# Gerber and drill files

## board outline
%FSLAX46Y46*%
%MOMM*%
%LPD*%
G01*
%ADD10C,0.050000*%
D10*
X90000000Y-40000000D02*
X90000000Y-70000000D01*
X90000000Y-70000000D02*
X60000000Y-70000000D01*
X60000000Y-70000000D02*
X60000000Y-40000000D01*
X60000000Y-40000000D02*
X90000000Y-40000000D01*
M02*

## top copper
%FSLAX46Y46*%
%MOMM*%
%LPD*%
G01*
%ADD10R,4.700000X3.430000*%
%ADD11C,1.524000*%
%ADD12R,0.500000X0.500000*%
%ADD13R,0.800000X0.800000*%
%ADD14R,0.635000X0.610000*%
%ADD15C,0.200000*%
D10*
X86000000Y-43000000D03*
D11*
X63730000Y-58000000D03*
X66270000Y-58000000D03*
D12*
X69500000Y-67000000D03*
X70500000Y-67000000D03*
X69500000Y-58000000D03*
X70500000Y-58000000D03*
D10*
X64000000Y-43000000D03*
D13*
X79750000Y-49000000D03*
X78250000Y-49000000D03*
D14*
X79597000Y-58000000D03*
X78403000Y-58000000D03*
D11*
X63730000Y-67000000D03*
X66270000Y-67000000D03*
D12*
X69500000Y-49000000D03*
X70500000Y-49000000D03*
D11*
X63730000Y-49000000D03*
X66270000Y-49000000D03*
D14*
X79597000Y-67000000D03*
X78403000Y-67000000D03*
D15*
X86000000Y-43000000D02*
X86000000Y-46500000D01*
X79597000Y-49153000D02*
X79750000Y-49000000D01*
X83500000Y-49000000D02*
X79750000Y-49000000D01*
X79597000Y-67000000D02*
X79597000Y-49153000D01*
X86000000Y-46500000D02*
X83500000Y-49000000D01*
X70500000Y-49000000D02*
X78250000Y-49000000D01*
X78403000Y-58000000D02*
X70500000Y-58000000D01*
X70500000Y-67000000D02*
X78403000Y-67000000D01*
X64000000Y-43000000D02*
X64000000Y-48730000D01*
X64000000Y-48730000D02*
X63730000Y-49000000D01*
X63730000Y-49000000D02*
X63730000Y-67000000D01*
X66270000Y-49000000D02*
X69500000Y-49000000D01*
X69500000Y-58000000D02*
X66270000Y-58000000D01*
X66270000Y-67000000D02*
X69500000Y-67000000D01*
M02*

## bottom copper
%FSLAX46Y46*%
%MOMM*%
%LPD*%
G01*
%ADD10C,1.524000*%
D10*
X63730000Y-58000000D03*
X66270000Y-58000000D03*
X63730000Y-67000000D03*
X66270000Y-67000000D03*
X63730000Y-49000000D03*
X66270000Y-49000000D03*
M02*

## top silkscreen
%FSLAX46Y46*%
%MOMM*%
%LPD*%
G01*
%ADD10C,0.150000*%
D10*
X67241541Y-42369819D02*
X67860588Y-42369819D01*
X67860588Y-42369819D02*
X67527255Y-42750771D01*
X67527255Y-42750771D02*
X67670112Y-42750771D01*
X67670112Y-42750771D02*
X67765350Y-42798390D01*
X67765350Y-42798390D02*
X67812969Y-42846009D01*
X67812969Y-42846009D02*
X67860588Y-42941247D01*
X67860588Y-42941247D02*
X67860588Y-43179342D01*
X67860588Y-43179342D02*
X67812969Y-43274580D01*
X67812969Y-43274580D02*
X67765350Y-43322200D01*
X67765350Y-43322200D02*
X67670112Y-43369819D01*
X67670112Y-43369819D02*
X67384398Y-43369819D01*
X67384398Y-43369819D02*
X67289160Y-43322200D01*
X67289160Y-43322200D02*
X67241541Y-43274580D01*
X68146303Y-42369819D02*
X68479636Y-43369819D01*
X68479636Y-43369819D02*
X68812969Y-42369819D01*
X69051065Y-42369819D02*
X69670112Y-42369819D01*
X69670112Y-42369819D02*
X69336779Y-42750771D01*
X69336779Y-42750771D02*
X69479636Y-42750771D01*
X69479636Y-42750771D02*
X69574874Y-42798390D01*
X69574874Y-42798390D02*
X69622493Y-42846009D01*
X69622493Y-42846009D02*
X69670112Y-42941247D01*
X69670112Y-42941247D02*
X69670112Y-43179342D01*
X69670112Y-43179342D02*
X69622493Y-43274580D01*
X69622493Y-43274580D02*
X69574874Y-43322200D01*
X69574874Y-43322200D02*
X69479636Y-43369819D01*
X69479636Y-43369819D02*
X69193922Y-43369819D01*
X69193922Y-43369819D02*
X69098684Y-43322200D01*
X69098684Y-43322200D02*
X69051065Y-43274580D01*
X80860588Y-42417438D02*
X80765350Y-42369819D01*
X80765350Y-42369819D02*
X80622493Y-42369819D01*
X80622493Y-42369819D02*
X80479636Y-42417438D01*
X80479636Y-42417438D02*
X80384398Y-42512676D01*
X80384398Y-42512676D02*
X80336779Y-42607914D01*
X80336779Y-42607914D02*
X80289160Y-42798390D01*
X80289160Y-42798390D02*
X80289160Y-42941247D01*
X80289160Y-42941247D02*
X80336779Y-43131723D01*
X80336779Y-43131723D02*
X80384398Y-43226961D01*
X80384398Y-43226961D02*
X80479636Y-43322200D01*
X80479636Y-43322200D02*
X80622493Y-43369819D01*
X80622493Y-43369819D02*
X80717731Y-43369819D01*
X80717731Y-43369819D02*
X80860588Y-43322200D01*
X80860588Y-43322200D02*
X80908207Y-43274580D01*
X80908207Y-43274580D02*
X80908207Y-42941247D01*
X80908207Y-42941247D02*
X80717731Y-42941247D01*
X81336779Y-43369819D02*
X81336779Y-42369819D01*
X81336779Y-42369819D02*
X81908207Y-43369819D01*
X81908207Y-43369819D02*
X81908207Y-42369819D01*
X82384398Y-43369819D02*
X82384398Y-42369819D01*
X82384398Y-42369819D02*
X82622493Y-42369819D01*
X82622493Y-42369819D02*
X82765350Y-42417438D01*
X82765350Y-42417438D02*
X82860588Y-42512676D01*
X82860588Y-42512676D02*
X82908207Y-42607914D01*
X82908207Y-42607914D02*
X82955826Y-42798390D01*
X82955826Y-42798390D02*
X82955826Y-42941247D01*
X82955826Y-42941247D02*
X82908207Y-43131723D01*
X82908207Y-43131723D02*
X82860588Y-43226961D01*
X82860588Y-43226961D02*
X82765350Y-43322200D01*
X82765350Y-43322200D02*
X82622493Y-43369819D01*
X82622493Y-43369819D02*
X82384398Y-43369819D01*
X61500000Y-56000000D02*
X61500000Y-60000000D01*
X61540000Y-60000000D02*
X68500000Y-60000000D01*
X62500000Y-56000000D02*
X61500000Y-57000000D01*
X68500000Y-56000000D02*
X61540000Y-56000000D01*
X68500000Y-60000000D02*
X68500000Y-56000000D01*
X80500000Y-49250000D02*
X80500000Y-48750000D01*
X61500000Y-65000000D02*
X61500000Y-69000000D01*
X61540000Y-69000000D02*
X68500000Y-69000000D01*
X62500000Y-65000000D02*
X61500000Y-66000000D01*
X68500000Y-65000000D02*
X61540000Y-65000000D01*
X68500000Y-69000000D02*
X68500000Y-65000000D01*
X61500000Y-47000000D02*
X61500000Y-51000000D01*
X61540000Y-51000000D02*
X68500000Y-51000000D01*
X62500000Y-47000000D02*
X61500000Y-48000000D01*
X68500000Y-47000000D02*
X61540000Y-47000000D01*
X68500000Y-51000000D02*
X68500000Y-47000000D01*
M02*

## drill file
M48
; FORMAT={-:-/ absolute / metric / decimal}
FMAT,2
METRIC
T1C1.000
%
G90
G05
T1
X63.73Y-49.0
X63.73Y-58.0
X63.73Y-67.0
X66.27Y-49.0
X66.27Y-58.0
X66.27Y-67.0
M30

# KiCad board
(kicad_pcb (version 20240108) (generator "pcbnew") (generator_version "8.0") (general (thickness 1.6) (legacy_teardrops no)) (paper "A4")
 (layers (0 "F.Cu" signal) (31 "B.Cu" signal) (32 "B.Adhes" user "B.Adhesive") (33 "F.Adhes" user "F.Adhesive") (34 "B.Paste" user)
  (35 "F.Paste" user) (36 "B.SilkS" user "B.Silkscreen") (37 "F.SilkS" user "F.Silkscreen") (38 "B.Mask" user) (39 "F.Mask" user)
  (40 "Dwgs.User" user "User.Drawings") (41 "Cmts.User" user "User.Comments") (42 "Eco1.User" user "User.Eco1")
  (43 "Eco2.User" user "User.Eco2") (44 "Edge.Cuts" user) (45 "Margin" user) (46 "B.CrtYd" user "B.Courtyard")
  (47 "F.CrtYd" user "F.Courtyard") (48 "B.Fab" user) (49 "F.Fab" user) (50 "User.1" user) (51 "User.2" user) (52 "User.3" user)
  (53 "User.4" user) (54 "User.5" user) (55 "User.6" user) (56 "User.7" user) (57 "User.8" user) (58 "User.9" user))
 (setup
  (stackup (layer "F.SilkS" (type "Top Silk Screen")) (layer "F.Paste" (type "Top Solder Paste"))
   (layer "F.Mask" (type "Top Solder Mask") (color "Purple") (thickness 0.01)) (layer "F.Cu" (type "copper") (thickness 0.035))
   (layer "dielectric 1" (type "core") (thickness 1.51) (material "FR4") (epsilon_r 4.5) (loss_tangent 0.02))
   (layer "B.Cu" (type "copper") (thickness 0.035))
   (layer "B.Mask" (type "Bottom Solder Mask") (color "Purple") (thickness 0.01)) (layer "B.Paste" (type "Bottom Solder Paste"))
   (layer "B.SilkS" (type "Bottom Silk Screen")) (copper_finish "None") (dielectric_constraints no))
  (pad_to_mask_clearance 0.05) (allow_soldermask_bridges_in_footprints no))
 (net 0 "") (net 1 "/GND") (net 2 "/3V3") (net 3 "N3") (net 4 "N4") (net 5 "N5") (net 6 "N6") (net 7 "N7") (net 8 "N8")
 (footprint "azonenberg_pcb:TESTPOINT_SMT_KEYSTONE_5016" (layer "F.Cu") (at 86 43)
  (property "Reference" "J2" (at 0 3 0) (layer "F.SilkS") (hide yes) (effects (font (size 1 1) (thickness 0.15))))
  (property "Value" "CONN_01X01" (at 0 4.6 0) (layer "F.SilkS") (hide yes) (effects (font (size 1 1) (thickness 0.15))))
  (pad "1" smd rect (at 0 0) (size 4.7 3.43) (layers "F.Cu" "F.Paste" "F.Mask") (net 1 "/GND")))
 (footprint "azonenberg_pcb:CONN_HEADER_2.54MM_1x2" (layer "F.Cu") (at 65 58)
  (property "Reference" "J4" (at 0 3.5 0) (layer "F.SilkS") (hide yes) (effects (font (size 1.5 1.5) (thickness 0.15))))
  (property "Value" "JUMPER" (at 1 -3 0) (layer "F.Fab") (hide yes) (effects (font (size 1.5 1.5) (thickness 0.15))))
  (fp_line (start -3.5 -2) (end -3.5 2) (stroke (width 0.15) (type solid)) (layer "F.SilkS"))
  (fp_line (start -3.46 2) (end 3.5 2) (stroke (width 0.15) (type solid)) (layer "F.SilkS"))
  (fp_line (start -2.5 -2) (end -3.5 -1) (stroke (width 0.15) (type solid)) (layer "F.SilkS"))
  (fp_line (start 3.5 -2) (end -3.46 -2) (stroke (width 0.15) (type solid)) (layer "F.SilkS"))
  (fp_line (start 3.5 2) (end 3.5 -2) (stroke (width 0.15) (type solid)) (layer "F.SilkS"))
  (pad "1" thru_hole circle (at -1.27 0) (size 1.524 1.524) (drill 1) (layers "*.Cu" "*.Mask") (remove_unused_layers no) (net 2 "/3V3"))
  (pad "2" thru_hole circle (at 1.27 0) (size 1.524 1.524) (drill 1) (layers "*.Cu" "*.Mask") (remove_unused_layers no) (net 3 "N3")))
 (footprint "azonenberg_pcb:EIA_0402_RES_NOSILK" (layer "F.Cu") (at 70 67)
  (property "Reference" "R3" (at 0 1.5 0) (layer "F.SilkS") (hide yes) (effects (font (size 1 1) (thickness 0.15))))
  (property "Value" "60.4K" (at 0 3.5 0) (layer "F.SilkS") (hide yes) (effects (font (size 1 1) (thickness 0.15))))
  (pad "1" smd rect (at -0.5 0) (size 0.5 0.5) (layers "F.Cu" "F.Paste" "F.Mask") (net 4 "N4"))
  (pad "2" smd rect (at 0.5 0) (size 0.5 0.5) (layers "F.Cu" "F.Paste" "F.Mask") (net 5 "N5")))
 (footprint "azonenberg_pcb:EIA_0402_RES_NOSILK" (layer "F.Cu") (at 70 58)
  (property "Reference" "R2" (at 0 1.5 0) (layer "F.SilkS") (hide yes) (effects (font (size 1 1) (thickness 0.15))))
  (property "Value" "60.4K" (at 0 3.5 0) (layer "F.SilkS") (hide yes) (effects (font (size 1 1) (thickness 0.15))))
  (pad "1" smd rect (at -0.5 0) (size 0.5 0.5) (layers "F.Cu" "F.Paste" "F.Mask") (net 3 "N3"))
  (pad "2" smd rect (at 0.5 0) (size 0.5 0.5) (layers "F.Cu" "F.Paste" "F.Mask") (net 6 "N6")))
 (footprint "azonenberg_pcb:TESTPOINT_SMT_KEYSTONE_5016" (layer "F.Cu") (at 64 43)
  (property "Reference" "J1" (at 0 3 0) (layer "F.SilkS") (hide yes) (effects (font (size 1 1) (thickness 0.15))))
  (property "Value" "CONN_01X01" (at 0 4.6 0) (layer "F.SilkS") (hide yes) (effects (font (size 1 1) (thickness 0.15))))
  (pad "1" smd rect (at 0 0) (size 4.7 3.43) (layers "F.Cu" "F.Paste" "F.Mask") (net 2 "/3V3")))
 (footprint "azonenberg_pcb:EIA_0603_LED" (layer "F.Cu") (at 79 49 180)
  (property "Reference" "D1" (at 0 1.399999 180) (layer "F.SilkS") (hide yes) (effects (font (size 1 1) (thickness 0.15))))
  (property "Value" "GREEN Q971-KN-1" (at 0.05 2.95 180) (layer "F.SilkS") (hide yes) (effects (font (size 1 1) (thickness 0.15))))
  (fp_line (start -1.5 -0.25) (end -1.5 0.25) (stroke (width 0.15) (type solid)) (layer "F.SilkS"))
  (pad "1" smd rect (at -0.75 0 180) (size 0.8 0.8) (layers "F.Cu" "F.Paste" "F.Mask") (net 1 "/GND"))
  (pad "2" smd rect (at 0.75 0 180) (size 0.8 0.8) (layers "F.Cu" "F.Paste" "F.Mask") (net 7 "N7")))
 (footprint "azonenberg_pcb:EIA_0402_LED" (layer "F.Cu") (at 79 58 180)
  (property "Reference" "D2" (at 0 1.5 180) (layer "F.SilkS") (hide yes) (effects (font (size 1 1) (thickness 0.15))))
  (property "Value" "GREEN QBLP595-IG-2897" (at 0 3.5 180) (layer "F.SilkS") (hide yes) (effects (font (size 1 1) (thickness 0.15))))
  (pad "1" smd rect (at -0.597 0 180) (size 0.635 0.61) (layers "F.Cu" "F.Paste" "F.Mask") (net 1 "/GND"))
  (pad "2" smd rect (at 0.597 0 180) (size 0.635 0.61) (layers "F.Cu" "F.Paste" "F.Mask") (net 6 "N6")))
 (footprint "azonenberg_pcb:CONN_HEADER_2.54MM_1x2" (layer "F.Cu") (at 65 67)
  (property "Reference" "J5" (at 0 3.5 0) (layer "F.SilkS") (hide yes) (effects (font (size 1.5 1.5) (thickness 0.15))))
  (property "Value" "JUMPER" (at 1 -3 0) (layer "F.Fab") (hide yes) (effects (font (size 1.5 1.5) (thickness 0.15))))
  (fp_line (start -3.5 -2) (end -3.5 2) (stroke (width 0.15) (type solid)) (layer "F.SilkS"))
  (fp_line (start -3.46 2) (end 3.5 2) (stroke (width 0.15) (type solid)) (layer "F.SilkS"))
  (fp_line (start -2.5 -2) (end -3.5 -1) (stroke (width 0.15) (type solid)) (layer "F.SilkS"))
  (fp_line (start 3.5 -2) (end -3.46 -2) (stroke (width 0.15) (type solid)) (layer "F.SilkS"))
  (fp_line (start 3.5 2) (end 3.5 -2) (stroke (width 0.15) (type solid)) (layer "F.SilkS"))
  (pad "1" thru_hole circle (at -1.27 0) (size 1.524 1.524) (drill 1) (layers "*.Cu" "*.Mask") (remove_unused_layers no) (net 2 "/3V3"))
  (pad "2" thru_hole circle (at 1.27 0) (size 1.524 1.524) (drill 1) (layers "*.Cu" "*.Mask") (remove_unused_layers no) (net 4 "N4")))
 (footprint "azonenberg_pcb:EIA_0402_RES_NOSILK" (layer "F.Cu") (at 70 49)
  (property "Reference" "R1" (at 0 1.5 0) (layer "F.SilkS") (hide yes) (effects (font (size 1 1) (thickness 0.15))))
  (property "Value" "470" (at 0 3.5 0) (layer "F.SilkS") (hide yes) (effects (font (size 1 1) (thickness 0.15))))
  (pad "1" smd rect (at -0.5 0) (size 0.5 0.5) (layers "F.Cu" "F.Paste" "F.Mask") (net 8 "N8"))
  (pad "2" smd rect (at 0.5 0) (size 0.5 0.5) (layers "F.Cu" "F.Paste" "F.Mask") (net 7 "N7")))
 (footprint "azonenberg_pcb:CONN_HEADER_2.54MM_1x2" (layer "F.Cu") (at 65 49)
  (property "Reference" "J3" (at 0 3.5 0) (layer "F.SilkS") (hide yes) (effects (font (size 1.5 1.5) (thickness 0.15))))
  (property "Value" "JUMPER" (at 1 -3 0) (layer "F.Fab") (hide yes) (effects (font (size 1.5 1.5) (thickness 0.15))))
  (fp_line (start -3.5 -2) (end -3.5 2) (stroke (width 0.15) (type solid)) (layer "F.SilkS"))
  (fp_line (start -3.46 2) (end 3.5 2) (stroke (width 0.15) (type solid)) (layer "F.SilkS"))
  (fp_line (start -2.5 -2) (end -3.5 -1) (stroke (width 0.15) (type solid)) (layer "F.SilkS"))
  (fp_line (start 3.5 -2) (end -3.46 -2) (stroke (width 0.15) (type solid)) (layer "F.SilkS"))
  (fp_line (start 3.5 2) (end 3.5 -2) (stroke (width 0.15) (type solid)) (layer "F.SilkS"))
  (pad "1" thru_hole circle (at -1.27 0) (size 1.524 1.524) (drill 1) (layers "*.Cu" "*.Mask") (remove_unused_layers no) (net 2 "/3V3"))
  (pad "2" thru_hole circle (at 1.27 0) (size 1.524 1.524) (drill 1) (layers "*.Cu" "*.Mask") (remove_unused_layers no) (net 8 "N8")))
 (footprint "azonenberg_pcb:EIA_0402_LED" (layer "F.Cu") (at 79 67 180)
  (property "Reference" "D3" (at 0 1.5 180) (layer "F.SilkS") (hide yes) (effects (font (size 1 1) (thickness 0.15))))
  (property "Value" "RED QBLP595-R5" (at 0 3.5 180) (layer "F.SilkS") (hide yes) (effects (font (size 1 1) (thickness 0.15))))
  (pad "1" smd rect (at -0.597 0 180) (size 0.635 0.61) (layers "F.Cu" "F.Paste" "F.Mask") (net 1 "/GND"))
  (pad "2" smd rect (at 0.597 0 180) (size 0.635 0.61) (layers "F.Cu" "F.Paste" "F.Mask") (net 5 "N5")))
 (gr_line (start 90 40) (end 90 70) (stroke (width 0.05) (type default)) (layer "Edge.Cuts"))
 (gr_line (start 90 70) (end 60 70) (stroke (width 0.05) (type default)) (layer "Edge.Cuts"))
 (gr_line (start 60 70) (end 60 40) (stroke (width 0.05) (type default)) (layer "Edge.Cuts"))
 (gr_line (start 60 40) (end 90 40) (stroke (width 0.05) (type default)) (layer "Edge.Cuts"))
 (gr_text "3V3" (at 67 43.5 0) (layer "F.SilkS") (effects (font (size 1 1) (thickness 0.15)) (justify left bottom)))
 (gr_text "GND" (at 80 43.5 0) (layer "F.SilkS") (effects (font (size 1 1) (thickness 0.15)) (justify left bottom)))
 (segment (start 86 43) (end 86 46.5) (width 0.2) (layer "F.Cu") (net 1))
 (segment (start 79.597 49.153) (end 79.75 49) (width 0.2) (layer "F.Cu") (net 1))
 (segment (start 83.5 49) (end 79.75 49) (width 0.2) (layer "F.Cu") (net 1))
 (segment (start 79.597 67) (end 79.597 49.153) (width 0.2) (layer "F.Cu") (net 1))
 (segment (start 86 46.5) (end 83.5 49) (width 0.2) (layer "F.Cu") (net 1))
 (segment (start 70.5 49) (end 78.25 49) (width 0.2) (layer "F.Cu") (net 7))
 (segment (start 78.403 58) (end 70.5 58) (width 0.2) (layer "F.Cu") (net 6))
 (segment (start 70.5 67) (end 78.403 67) (width 0.2) (layer "F.Cu") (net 5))
 (segment (start 64 43) (end 64 48.73) (width 0.2) (layer "F.Cu") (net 2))
 (segment (start 64 48.73) (end 63.73 49) (width 0.2) (layer "F.Cu") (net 2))
 (segment (start 63.73 49) (end 63.73 67) (width 0.2) (layer "F.Cu") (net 2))
 (segment (start 66.27 49) (end 69.5 49) (width 0.2) (layer "F.Cu") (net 8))
 (segment (start 69.5 58) (end 66.27 58) (width 0.2) (layer "F.Cu") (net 3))
 (segment (start 66.27 67) (end 69.5 67) (width 0.2) (layer "F.Cu") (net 4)))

